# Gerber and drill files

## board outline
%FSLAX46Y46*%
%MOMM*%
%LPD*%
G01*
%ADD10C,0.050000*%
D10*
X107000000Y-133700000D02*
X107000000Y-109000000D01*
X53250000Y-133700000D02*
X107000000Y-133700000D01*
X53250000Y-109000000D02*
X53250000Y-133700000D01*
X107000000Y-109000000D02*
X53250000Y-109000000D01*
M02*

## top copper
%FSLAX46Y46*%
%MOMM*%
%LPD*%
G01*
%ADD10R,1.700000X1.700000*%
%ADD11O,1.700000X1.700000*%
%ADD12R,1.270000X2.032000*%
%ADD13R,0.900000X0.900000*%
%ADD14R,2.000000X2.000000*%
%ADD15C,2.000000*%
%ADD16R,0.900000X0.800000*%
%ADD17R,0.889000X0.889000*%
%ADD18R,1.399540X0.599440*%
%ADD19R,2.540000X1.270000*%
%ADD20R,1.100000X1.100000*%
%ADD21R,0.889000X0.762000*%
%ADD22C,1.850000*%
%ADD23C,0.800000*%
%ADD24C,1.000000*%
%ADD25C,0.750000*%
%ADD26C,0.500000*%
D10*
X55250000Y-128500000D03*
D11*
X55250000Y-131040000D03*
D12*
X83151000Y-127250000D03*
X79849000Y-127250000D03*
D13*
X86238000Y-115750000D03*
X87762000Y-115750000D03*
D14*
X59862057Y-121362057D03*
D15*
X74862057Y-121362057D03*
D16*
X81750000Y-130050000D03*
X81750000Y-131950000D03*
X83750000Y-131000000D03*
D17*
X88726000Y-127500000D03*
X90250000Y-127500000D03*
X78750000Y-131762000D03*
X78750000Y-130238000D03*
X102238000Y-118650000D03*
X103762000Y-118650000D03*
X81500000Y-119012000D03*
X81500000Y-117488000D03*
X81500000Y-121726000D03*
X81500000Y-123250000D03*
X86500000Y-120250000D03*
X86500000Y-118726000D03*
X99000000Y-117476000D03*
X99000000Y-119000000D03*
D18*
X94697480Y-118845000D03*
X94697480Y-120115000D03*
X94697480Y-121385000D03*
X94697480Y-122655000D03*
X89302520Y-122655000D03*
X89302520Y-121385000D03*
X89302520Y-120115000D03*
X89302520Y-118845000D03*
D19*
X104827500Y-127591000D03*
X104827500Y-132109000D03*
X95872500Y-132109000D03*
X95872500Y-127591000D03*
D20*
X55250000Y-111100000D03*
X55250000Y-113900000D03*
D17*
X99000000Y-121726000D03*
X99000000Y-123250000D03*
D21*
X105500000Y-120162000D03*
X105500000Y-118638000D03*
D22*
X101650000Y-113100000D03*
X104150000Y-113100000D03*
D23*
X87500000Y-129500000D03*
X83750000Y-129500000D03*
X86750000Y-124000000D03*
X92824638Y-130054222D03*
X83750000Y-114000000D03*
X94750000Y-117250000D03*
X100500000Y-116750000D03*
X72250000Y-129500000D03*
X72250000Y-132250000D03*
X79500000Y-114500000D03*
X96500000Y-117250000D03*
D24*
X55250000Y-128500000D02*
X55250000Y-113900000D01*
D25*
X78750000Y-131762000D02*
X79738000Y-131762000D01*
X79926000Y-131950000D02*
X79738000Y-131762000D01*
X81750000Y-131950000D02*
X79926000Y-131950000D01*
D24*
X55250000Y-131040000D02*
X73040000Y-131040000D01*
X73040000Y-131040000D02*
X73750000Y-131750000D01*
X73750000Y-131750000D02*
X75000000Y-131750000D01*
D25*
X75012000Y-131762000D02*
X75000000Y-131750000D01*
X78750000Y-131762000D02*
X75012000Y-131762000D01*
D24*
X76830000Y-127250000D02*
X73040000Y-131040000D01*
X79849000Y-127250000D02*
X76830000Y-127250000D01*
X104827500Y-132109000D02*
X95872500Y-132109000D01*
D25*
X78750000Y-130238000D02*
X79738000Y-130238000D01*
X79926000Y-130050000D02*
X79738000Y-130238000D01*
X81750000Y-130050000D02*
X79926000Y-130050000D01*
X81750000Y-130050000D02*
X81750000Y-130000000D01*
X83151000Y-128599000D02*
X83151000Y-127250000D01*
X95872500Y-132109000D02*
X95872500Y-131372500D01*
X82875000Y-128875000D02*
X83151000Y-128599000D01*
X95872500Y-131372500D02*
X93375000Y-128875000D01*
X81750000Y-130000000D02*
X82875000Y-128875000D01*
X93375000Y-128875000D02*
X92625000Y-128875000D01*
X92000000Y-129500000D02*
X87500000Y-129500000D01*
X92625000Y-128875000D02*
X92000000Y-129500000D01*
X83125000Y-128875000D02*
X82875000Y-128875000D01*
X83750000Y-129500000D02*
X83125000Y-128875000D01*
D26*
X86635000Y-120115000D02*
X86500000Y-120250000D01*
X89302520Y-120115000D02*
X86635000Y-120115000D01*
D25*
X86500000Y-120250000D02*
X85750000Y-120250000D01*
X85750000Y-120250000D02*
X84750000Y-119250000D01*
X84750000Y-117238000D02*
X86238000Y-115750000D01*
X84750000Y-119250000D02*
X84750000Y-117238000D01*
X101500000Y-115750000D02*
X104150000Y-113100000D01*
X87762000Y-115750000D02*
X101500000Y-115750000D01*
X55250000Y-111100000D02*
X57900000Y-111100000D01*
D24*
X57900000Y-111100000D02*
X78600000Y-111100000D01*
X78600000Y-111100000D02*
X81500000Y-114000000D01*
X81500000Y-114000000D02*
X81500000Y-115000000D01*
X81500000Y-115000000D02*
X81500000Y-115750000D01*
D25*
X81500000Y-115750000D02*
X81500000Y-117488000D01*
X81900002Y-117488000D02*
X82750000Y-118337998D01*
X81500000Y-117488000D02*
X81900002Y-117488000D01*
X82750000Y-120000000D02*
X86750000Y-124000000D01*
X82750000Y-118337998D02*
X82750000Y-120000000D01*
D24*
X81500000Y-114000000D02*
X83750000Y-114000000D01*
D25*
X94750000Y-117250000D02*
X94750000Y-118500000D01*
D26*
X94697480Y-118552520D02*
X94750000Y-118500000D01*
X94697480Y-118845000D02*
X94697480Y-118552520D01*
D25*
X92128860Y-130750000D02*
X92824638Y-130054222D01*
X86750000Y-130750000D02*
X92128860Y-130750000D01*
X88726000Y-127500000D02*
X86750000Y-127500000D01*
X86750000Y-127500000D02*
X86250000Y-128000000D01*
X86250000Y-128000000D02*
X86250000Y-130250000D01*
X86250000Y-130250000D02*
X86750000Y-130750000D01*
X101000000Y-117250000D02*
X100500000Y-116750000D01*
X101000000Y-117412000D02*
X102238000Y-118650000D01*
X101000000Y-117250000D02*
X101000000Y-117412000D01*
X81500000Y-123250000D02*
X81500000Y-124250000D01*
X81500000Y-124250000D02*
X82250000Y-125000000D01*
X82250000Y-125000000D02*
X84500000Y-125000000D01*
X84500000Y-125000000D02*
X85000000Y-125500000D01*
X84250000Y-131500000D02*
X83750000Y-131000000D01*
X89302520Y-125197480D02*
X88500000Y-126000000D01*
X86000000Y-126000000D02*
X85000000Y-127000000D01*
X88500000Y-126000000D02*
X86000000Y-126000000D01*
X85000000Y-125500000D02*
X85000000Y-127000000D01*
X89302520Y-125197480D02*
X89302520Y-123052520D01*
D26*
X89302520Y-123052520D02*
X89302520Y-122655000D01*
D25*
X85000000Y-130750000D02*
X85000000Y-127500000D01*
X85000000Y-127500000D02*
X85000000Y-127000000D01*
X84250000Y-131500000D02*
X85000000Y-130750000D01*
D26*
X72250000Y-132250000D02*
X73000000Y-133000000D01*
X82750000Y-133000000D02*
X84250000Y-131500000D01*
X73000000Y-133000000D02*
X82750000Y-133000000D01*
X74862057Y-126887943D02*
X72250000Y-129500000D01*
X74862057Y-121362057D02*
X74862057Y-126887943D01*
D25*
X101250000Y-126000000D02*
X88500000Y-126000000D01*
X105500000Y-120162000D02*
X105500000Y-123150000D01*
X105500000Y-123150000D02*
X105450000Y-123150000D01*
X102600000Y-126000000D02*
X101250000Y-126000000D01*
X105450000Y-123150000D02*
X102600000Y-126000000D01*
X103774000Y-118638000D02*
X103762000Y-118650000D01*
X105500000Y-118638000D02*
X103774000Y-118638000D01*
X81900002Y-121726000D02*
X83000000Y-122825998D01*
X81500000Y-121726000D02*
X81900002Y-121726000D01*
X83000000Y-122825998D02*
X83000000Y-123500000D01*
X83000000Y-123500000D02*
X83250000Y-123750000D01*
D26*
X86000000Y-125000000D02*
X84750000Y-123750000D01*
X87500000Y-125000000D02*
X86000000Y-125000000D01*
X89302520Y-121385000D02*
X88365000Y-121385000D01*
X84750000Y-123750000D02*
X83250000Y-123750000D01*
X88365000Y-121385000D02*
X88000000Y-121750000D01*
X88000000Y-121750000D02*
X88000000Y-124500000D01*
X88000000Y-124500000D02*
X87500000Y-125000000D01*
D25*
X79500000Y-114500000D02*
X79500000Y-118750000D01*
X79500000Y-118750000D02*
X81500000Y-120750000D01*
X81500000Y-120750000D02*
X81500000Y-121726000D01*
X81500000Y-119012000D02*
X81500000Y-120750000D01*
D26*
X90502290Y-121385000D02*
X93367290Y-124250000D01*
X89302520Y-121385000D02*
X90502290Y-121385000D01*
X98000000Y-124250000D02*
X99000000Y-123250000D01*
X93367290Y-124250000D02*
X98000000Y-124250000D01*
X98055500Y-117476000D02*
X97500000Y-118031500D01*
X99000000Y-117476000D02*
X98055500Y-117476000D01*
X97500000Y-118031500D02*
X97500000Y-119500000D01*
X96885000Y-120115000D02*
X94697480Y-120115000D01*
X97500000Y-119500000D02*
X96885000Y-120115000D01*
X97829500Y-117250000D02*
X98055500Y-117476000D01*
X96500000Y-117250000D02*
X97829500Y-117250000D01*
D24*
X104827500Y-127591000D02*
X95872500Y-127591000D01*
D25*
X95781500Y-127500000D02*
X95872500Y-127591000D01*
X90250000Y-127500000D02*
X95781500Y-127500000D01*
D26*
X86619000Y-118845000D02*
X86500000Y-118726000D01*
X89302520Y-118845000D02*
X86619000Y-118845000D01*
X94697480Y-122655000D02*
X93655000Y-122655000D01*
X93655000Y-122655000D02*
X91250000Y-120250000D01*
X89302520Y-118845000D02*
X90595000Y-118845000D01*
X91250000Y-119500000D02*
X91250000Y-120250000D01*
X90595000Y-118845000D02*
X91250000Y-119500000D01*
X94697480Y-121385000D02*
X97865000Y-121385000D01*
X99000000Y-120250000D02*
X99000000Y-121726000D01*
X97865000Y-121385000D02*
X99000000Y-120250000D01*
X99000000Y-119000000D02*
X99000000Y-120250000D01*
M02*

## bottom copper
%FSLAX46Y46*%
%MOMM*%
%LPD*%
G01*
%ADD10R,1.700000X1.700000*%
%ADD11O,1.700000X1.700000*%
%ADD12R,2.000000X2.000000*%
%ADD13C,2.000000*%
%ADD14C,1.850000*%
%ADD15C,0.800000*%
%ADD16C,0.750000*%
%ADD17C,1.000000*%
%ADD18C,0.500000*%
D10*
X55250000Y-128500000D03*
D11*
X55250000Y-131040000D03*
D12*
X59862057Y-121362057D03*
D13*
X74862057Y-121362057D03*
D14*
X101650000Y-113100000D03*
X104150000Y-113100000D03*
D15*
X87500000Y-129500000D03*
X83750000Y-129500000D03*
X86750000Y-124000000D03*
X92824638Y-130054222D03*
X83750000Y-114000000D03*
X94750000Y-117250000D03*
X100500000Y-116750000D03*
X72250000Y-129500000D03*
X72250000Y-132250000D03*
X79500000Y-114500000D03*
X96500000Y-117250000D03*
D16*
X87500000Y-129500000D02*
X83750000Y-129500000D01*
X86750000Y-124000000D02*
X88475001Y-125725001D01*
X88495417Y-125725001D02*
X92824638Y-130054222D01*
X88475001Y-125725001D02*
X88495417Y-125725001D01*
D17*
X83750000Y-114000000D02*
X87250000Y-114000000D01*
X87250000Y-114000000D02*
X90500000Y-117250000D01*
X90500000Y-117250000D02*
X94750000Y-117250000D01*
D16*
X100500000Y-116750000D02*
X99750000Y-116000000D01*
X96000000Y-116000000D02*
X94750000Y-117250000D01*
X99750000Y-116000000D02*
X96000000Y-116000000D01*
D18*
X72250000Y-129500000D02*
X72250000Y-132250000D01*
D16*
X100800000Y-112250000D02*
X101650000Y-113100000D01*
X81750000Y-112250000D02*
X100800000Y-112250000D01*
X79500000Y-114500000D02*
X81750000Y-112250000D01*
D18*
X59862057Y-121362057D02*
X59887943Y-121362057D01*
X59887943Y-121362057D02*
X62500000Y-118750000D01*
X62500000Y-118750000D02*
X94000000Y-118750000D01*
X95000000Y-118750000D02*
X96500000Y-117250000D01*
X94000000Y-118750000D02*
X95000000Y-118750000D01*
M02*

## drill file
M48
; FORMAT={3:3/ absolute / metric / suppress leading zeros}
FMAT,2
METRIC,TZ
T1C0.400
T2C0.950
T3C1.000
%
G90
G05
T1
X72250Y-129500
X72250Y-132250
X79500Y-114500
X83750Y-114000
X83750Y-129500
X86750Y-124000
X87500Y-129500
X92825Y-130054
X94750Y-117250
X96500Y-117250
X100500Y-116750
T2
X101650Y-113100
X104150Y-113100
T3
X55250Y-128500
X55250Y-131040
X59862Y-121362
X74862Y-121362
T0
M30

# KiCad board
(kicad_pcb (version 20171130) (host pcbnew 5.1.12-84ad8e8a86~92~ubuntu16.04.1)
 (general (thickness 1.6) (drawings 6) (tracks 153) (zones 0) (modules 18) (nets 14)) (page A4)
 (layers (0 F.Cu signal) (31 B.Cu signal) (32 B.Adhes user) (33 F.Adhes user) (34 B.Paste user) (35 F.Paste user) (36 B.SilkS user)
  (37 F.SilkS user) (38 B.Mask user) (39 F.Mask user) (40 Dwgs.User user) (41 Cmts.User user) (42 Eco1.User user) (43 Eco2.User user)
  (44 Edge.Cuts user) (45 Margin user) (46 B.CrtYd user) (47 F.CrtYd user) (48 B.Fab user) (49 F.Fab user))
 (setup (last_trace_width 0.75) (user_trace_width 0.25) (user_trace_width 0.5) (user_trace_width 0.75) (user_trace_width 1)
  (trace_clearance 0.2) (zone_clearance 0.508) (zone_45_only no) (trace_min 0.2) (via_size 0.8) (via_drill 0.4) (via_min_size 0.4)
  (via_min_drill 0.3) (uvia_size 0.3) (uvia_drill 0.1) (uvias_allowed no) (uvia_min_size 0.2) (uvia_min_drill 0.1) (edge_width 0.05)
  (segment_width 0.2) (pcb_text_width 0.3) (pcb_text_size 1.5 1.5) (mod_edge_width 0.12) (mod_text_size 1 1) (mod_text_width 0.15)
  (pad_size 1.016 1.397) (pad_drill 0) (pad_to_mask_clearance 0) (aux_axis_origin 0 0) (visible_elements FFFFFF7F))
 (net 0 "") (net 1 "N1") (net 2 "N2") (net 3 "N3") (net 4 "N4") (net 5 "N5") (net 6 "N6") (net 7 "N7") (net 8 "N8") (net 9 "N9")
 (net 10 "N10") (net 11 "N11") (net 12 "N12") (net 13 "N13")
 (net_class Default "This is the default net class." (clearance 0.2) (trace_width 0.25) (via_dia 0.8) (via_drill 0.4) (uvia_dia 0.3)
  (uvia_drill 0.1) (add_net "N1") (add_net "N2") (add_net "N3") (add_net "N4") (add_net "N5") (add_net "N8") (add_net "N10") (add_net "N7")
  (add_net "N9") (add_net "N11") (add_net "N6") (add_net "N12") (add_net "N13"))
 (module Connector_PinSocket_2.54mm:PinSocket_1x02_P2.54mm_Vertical (layer F.Cu) (at 55.25 128.5)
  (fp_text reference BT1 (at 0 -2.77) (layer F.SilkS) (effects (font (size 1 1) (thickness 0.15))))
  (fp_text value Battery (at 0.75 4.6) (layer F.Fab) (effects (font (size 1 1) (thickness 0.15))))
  (pad 1 thru_hole rect (at 0 0) (size 1.7 1.7) (drill 1) (layers *.Cu *.Mask) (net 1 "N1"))
  (pad 2 thru_hole oval (at 0 2.54) (size 1.7 1.7) (drill 1) (layers *.Cu *.Mask) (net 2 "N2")))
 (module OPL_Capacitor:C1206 (layer F.Cu) (at 81.5 127.25 180)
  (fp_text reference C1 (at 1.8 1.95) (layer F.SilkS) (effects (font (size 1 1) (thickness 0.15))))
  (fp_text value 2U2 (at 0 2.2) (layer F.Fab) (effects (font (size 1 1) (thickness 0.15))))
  (pad 1 smd rect (at -1.651 0 180) (size 1.27 2.032) (layers F.Cu F.Paste F.Mask) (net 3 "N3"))
  (pad 2 smd rect (at 1.651 0 180) (size 1.27 2.032) (layers F.Cu F.Paste F.Mask) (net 2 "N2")))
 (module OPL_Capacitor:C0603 (layer F.Cu) (at 87 115.75)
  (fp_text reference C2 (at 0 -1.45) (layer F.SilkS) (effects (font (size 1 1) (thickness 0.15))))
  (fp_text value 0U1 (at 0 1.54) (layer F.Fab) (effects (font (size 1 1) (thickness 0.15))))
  (pad 1 smd rect (at -0.762 0) (size 0.9 0.9) (layers F.Cu F.Paste F.Mask) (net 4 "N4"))
  (pad 2 smd rect (at 0.762 0) (size 0.9 0.9) (layers F.Cu F.Paste F.Mask) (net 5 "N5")))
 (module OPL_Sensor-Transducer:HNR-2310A (layer F.Cu) (at 59.862057 121.362057)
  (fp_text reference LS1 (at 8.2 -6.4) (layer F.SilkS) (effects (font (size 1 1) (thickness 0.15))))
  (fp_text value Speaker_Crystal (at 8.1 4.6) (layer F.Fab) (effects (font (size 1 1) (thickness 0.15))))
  (pad 1 thru_hole rect (at 0 0) (size 2 2) (drill 1) (layers *.Cu *.Mask) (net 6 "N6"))
  (pad 2 thru_hole circle (at 15 0) (size 2 2) (drill 1) (layers *.Cu *.Mask) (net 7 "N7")))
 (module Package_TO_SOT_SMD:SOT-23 (layer F.Cu) (at 82.75 131)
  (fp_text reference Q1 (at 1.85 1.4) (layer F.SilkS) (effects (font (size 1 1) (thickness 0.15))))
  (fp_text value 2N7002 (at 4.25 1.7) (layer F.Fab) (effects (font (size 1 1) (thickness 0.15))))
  (pad 1 smd rect (at -1 -0.95) (size 0.9 0.8) (layers F.Cu F.Paste F.Mask) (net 3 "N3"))
  (pad 2 smd rect (at -1 0.95) (size 0.9 0.8) (layers F.Cu F.Paste F.Mask) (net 2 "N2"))
  (pad 3 smd rect (at 1 0) (size 0.9 0.8) (layers F.Cu F.Paste F.Mask) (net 7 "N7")))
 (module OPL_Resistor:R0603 (layer F.Cu) (at 89.488 127.5)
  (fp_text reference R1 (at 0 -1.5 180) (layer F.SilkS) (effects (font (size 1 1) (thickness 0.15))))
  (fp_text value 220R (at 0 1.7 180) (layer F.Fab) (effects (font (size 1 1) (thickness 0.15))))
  (pad 1 smd rect (at -0.762 0) (size 0.889 0.889) (layers F.Cu F.Paste F.Mask) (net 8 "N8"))
  (pad 2 smd rect (at 0.762 0) (size 0.889 0.889) (layers F.Cu F.Paste F.Mask) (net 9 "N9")))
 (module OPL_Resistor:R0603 (layer F.Cu) (at 78.75 131 270)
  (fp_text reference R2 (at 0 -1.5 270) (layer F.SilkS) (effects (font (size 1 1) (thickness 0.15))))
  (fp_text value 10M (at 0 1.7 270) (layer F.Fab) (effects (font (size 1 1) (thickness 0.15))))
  (pad 2 smd rect (at 0.762 0 270) (size 0.889 0.889) (layers F.Cu F.Paste F.Mask) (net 2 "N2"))
  (pad 1 smd rect (at -0.762 0 270) (size 0.889 0.889) (layers F.Cu F.Paste F.Mask) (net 3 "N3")))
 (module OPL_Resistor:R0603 (layer F.Cu) (at 103 118.65)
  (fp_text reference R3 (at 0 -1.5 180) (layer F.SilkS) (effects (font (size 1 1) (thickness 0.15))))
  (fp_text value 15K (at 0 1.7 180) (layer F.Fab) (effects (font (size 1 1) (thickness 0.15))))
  (pad 1 smd rect (at -0.762 0) (size 0.889 0.889) (layers F.Cu F.Paste F.Mask) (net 8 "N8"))
  (pad 2 smd rect (at 0.762 0) (size 0.889 0.889) (layers F.Cu F.Paste F.Mask) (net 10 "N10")))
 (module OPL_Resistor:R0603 (layer F.Cu) (at 81.5 118.25 270)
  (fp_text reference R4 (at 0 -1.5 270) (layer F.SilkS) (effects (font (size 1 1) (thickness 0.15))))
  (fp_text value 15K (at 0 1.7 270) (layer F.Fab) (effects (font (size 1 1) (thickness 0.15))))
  (pad 2 smd rect (at 0.762 0 270) (size 0.889 0.889) (layers F.Cu F.Paste F.Mask) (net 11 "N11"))
  (pad 1 smd rect (at -0.762 0 270) (size 0.889 0.889) (layers F.Cu F.Paste F.Mask) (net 8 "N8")))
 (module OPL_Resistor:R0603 (layer F.Cu) (at 81.5 122.488 270)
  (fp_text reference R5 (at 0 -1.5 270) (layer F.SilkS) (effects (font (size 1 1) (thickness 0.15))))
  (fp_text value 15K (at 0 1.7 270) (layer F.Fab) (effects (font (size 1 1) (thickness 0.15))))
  (pad 1 smd rect (at -0.762 0 270) (size 0.889 0.889) (layers F.Cu F.Paste F.Mask) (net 11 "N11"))
  (pad 2 smd rect (at 0.762 0 270) (size 0.889 0.889) (layers F.Cu F.Paste F.Mask) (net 7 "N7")))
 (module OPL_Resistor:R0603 (layer F.Cu) (at 86.5 119.488 270)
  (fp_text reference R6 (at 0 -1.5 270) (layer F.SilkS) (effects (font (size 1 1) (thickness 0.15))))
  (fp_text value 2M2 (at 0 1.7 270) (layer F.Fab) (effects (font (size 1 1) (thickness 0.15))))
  (pad 2 smd rect (at 0.762 0 270) (size 0.889 0.889) (layers F.Cu F.Paste F.Mask) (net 4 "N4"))
  (pad 1 smd rect (at -0.762 0 270) (size 0.889 0.889) (layers F.Cu F.Paste F.Mask) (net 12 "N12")))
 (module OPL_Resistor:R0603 (layer F.Cu) (at 99 118.238 270)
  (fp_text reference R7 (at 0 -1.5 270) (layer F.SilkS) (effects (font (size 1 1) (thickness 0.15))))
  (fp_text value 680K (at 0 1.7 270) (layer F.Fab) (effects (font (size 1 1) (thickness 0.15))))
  (pad 1 smd rect (at -0.762 0 270) (size 0.889 0.889) (layers F.Cu F.Paste F.Mask) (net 6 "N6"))
  (pad 2 smd rect (at 0.762 0 270) (size 0.889 0.889) (layers F.Cu F.Paste F.Mask) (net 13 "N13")))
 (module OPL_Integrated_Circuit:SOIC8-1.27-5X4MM (layer F.Cu) (at 92 120.75)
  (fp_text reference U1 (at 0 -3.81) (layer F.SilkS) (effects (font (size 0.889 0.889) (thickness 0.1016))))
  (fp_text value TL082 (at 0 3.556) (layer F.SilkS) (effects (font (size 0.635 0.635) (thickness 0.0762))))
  (pad 8 smd rect (at 2.69748 -1.905) (size 1.39954 0.59944) (layers F.Cu F.Paste F.Mask) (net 8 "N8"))
  (pad 7 smd rect (at 2.69748 -0.635) (size 1.39954 0.59944) (layers F.Cu F.Paste F.Mask) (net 6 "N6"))
  (pad 6 smd rect (at 2.69748 0.635) (size 1.39954 0.59944) (layers F.Cu F.Paste F.Mask) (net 13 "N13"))
  (pad 5 smd rect (at 2.69748 1.905) (size 1.39954 0.59944) (layers F.Cu F.Paste F.Mask) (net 12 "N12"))
  (pad 4 smd rect (at -2.69748 1.905) (size 1.39954 0.59944) (layers F.Cu F.Paste F.Mask) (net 7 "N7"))
  (pad 3 smd rect (at -2.69748 0.635) (size 1.39954 0.59944) (layers F.Cu F.Paste F.Mask) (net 11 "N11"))
  (pad 2 smd rect (at -2.69748 -0.635) (size 1.39954 0.59944) (layers F.Cu F.Paste F.Mask) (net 4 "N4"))
  (pad 1 smd rect (at -2.69748 -1.905) (size 1.39954 0.59944) (layers F.Cu F.Paste F.Mask) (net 12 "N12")))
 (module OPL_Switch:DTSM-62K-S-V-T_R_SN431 (layer F.Cu) (at 100 129.75)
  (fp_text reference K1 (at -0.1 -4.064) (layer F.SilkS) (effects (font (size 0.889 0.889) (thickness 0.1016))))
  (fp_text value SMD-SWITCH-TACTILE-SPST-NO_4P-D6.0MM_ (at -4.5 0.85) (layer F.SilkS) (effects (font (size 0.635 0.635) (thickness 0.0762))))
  (pad 4 smd rect (at 4.8275 -2.159) (size 2.54 1.27) (layers F.Cu F.Paste F.Mask) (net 9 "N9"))
  (pad 3 smd rect (at 4.8275 2.359) (size 2.54 1.27) (layers F.Cu F.Paste F.Mask) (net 3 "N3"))
  (pad 2 smd rect (at -4.1275 2.359) (size 2.54 1.27) (layers F.Cu F.Paste F.Mask) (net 3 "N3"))
  (pad 1 smd rect (at -4.1275 -2.159) (size 2.54 1.27) (layers F.Cu F.Paste F.Mask) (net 9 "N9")))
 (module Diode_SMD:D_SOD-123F (layer F.Cu) (at 55.25 112.5 270)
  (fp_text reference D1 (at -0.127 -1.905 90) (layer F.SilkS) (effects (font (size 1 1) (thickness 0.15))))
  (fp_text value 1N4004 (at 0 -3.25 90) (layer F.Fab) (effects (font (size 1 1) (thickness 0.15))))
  (pad 1 smd rect (at -1.4 0 270) (size 1.1 1.1) (layers F.Cu F.Paste F.Mask) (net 8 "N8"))
  (pad 2 smd rect (at 1.4 0 270) (size 1.1 1.1) (layers F.Cu F.Paste F.Mask) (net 1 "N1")))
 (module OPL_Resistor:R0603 (layer F.Cu) (at 99 122.488 270)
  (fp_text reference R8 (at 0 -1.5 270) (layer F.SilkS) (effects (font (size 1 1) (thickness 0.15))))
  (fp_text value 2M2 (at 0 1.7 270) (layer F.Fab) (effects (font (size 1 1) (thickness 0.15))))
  (pad 1 smd rect (at -0.762 0 270) (size 0.889 0.889) (layers F.Cu F.Paste F.Mask) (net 13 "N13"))
  (pad 2 smd rect (at 0.762 0 270) (size 0.889 0.889) (layers F.Cu F.Paste F.Mask) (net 11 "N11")))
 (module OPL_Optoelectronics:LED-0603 (layer F.Cu) (at 105.5 119.4 270)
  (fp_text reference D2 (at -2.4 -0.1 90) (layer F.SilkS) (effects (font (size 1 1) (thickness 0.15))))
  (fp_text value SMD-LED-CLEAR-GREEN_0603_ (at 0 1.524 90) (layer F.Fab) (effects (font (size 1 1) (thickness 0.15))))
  (pad 2 smd rect (at 0.762 0 270) (size 0.762 0.889) (layers F.Cu F.Paste F.Mask) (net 7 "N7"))
  (pad 1 smd rect (at -0.762 0 270) (size 0.762 0.889) (layers F.Cu F.Paste F.Mask) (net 10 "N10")))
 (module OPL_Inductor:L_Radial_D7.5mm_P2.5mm (layer F.Cu) (at 100.9 113.1)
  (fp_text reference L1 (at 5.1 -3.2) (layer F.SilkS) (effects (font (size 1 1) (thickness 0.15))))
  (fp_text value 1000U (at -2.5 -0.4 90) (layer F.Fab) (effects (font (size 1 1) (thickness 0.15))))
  (pad 1 thru_hole circle (at 0.75 0) (size 1.85 1.85) (drill 0.95) (layers *.Cu *.Mask) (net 11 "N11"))
  (pad 2 thru_hole circle (at 3.25 0) (size 1.85 1.85) (drill 0.95) (layers *.Cu *.Mask) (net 5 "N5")))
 (gr_line (start 107 133.7) (end 107 109) (layer Edge.Cuts) (width 0.05))
 (gr_line (start 53.25 133.7) (end 107 133.7) (layer Edge.Cuts) (width 0.05))
 (gr_line (start 53.25 109) (end 53.25 133.7) (layer Edge.Cuts) (width 0.05))
 (gr_line (start 107 109) (end 53.25 109) (layer Edge.Cuts) (width 0.05))
 (segment (start 55.25 128.5) (end 55.25 113.9) (width 1) (layer F.Cu) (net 1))
 (segment (start 78.75 131.762) (end 79.738 131.762) (width 0.75) (layer F.Cu) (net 2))
 (segment (start 79.926 131.95) (end 79.738 131.762) (width 0.75) (layer F.Cu) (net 2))
 (segment (start 81.75 131.95) (end 79.926 131.95) (width 0.75) (layer F.Cu) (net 2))
 (segment (start 55.25 131.04) (end 73.04 131.04) (width 1) (layer F.Cu) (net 2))
 (segment (start 73.04 131.04) (end 73.75 131.75) (width 1) (layer F.Cu) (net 2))
 (segment (start 73.75 131.75) (end 75 131.75) (width 1) (layer F.Cu) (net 2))
 (segment (start 75.012 131.762) (end 75 131.75) (width 0.75) (layer F.Cu) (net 2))
 (segment (start 78.75 131.762) (end 75.012 131.762) (width 0.75) (layer F.Cu) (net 2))
 (segment (start 76.83 127.25) (end 73.04 131.04) (width 1) (layer F.Cu) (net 2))
 (segment (start 79.849 127.25) (end 76.83 127.25) (width 1) (layer F.Cu) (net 2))
 (segment (start 104.8275 132.109) (end 95.8725 132.109) (width 1) (layer F.Cu) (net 3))
 (segment (start 78.75 130.238) (end 79.738 130.238) (width 0.75) (layer F.Cu) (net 3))
 (segment (start 79.926 130.05) (end 79.738 130.238) (width 0.75) (layer F.Cu) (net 3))
 (segment (start 81.75 130.05) (end 79.926 130.05) (width 0.75) (layer F.Cu) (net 3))
 (segment (start 81.75 130.05) (end 81.75 130) (width 0.75) (layer F.Cu) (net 3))
 (segment (start 83.151 128.599) (end 83.151 127.25) (width 0.75) (layer F.Cu) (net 3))
 (segment (start 95.8725 132.109) (end 95.8725 131.3725) (width 0.75) (layer F.Cu) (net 3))
 (segment (start 82.875 128.875) (end 83.151 128.599) (width 0.75) (layer F.Cu) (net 3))
 (segment (start 95.8725 131.3725) (end 93.375 128.875) (width 0.75) (layer F.Cu) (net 3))
 (segment (start 81.75 130) (end 82.875 128.875) (width 0.75) (layer F.Cu) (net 3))
 (segment (start 93.375 128.875) (end 92.625 128.875) (width 0.75) (layer F.Cu) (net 3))
 (segment (start 92 129.5) (end 87.5 129.5) (width 0.75) (layer F.Cu) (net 3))
 (via (at 87.5 129.5) (size 0.8) (drill 0.4) (layers F.Cu B.Cu) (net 3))
 (segment (start 92.625 128.875) (end 92 129.5) (width 0.75) (layer F.Cu) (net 3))
 (via (at 83.75 129.5) (size 0.8) (drill 0.4) (layers F.Cu B.Cu) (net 3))
 (segment (start 87.5 129.5) (end 83.75 129.5) (width 0.75) (layer B.Cu) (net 3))
 (segment (start 83.125 128.875) (end 82.875 128.875) (width 0.75) (layer F.Cu) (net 3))
 (segment (start 83.75 129.5) (end 83.125 128.875) (width 0.75) (layer F.Cu) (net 3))
 (segment (start 86.635 120.115) (end 86.5 120.25) (width 0.5) (layer F.Cu) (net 4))
 (segment (start 89.30252 120.115) (end 86.635 120.115) (width 0.5) (layer F.Cu) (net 4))
 (segment (start 86.5 120.25) (end 85.75 120.25) (width 0.75) (layer F.Cu) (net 4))
 (segment (start 85.75 120.25) (end 84.75 119.25) (width 0.75) (layer F.Cu) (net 4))
 (segment (start 84.75 117.238) (end 86.238 115.75) (width 0.75) (layer F.Cu) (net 4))
 (segment (start 84.75 119.25) (end 84.75 117.238) (width 0.75) (layer F.Cu) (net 4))
 (segment (start 101.5 115.75) (end 104.15 113.1) (width 0.75) (layer F.Cu) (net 5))
 (segment (start 87.762 115.75) (end 101.5 115.75) (width 0.75) (layer F.Cu) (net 5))
 (segment (start 55.25 111.1) (end 57.9 111.1) (width 0.75) (layer F.Cu) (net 8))
 (segment (start 57.9 111.1) (end 78.6 111.1) (width 1) (layer F.Cu) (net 8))
 (segment (start 78.6 111.1) (end 81.5 114) (width 1) (layer F.Cu) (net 8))
 (segment (start 81.5 114) (end 81.5 115) (width 1) (layer F.Cu) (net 8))
 (segment (start 81.5 115) (end 81.5 115.75) (width 1) (layer F.Cu) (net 8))
 (segment (start 81.5 115.75) (end 81.5 117.488) (width 0.75) (layer F.Cu) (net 8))
 (segment (start 81.900002 117.488) (end 82.75 118.337998) (width 0.75) (layer F.Cu) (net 8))
 (segment (start 81.5 117.488) (end 81.900002 117.488) (width 0.75) (layer F.Cu) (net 8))
 (segment (start 82.75 120) (end 86.75 124) (width 0.75) (layer F.Cu) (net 8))
 (via (at 86.75 124) (size 0.8) (drill 0.4) (layers F.Cu B.Cu) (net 8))
 (segment (start 82.75 118.337998) (end 82.75 120) (width 0.75) (layer F.Cu) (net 8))
 (segment (start 86.75 124) (end 88.475001 125.725001) (width 0.75) (layer B.Cu) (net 8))
 (via (at 92.824638 130.054222) (size 0.8) (drill 0.4) (layers F.Cu B.Cu) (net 8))
 (segment (start 88.495417 125.725001) (end 92.824638 130.054222) (width 0.75) (layer B.Cu) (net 8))
 (segment (start 88.475001 125.725001) (end 88.495417 125.725001) (width 0.75) (layer B.Cu) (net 8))
 (via (at 83.75 114) (size 0.8) (drill 0.4) (layers F.Cu B.Cu) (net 8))
 (segment (start 81.5 114) (end 83.75 114) (width 1) (layer F.Cu) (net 8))
 (segment (start 83.75 114) (end 87.25 114) (width 1) (layer B.Cu) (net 8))
 (segment (start 87.25 114) (end 90.5 117.25) (width 1) (layer B.Cu) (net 8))
 (via (at 94.75 117.25) (size 0.8) (drill 0.4) (layers F.Cu B.Cu) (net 8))
 (segment (start 90.5 117.25) (end 94.75 117.25) (width 1) (layer B.Cu) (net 8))
 (segment (start 94.75 117.25) (end 94.75 118.5) (width 0.75) (layer F.Cu) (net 8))
 (segment (start 94.69748 118.55252) (end 94.75 118.5) (width 0.5) (layer F.Cu) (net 8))
 (segment (start 94.69748 118.845) (end 94.69748 118.55252) (width 0.5) (layer F.Cu) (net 8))
 (segment (start 92.12886 130.75) (end 92.824638 130.054222) (width 0.75) (layer F.Cu) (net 8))
 (segment (start 86.75 130.75) (end 92.12886 130.75) (width 0.75) (layer F.Cu) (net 8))
 (segment (start 88.726 127.5) (end 86.75 127.5) (width 0.75) (layer F.Cu) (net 8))
 (segment (start 86.75 127.5) (end 86.25 128) (width 0.75) (layer F.Cu) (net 8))
 (segment (start 86.25 128) (end 86.25 130.25) (width 0.75) (layer F.Cu) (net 8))
 (segment (start 86.25 130.25) (end 86.75 130.75) (width 0.75) (layer F.Cu) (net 8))
 (via (at 100.5 116.75) (size 0.8) (drill 0.4) (layers F.Cu B.Cu) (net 8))
 (segment (start 101 117.25) (end 100.5 116.75) (width 0.75) (layer F.Cu) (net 8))
 (segment (start 100.5 116.75) (end 99.75 116) (width 0.75) (layer B.Cu) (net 8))
 (segment (start 96 116) (end 94.75 117.25) (width 0.75) (layer B.Cu) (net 8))
 (segment (start 99.75 116) (end 96 116) (width 0.75) (layer B.Cu) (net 8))
 (segment (start 101 117.412) (end 102.238 118.65) (width 0.75) (layer F.Cu) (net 8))
 (segment (start 101 117.25) (end 101 117.412) (width 0.75) (layer F.Cu) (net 8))
 (segment (start 81.5 123.25) (end 81.5 124.25) (width 0.75) (layer F.Cu) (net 7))
 (segment (start 81.5 124.25) (end 82.25 125) (width 0.75) (layer F.Cu) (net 7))
 (segment (start 82.25 125) (end 84.5 125) (width 0.75) (layer F.Cu) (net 7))
 (segment (start 84.5 125) (end 85 125.5) (width 0.75) (layer F.Cu) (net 7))
 (segment (start 84.25 131.5) (end 83.75 131) (width 0.75) (layer F.Cu) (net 7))
 (segment (start 89.30252 125.19748) (end 88.5 126) (width 0.75) (layer F.Cu) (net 7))
 (segment (start 86 126) (end 85 127) (width 0.75) (layer F.Cu) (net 7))
 (segment (start 88.5 126) (end 86 126) (width 0.75) (layer F.Cu) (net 7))
 (segment (start 85 125.5) (end 85 127) (width 0.75) (layer F.Cu) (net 7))
 (segment (start 89.30252 125.19748) (end 89.30252 123.05252) (width 0.75) (layer F.Cu) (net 7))
 (segment (start 89.30252 123.05252) (end 89.30252 122.655) (width 0.5) (layer F.Cu) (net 7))
 (segment (start 85 130.75) (end 85 127.5) (width 0.75) (layer F.Cu) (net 7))
 (segment (start 85 127.5) (end 85 127) (width 0.75) (layer F.Cu) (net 7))
 (segment (start 84.25 131.5) (end 85 130.75) (width 0.75) (layer F.Cu) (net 7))
 (via (at 72.25 129.5) (size 0.8) (drill 0.4) (layers F.Cu B.Cu) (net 7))
 (via (at 72.25 132.25) (size 0.8) (drill 0.4) (layers F.Cu B.Cu) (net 7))
 (segment (start 72.25 132.25) (end 73 133) (width 0.5) (layer F.Cu) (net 7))
 (segment (start 82.75 133) (end 84.25 131.5) (width 0.5) (layer F.Cu) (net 7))
 (segment (start 73 133) (end 82.75 133) (width 0.5) (layer F.Cu) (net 7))
 (segment (start 74.862057 126.887943) (end 72.25 129.5) (width 0.5) (layer F.Cu) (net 7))
 (segment (start 74.862057 121.362057) (end 74.862057 126.887943) (width 0.5) (layer F.Cu) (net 7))
 (segment (start 72.25 129.5) (end 72.25 132.25) (width 0.5) (layer B.Cu) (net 7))
 (segment (start 101.25 126) (end 88.5 126) (width 0.75) (layer F.Cu) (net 7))
 (segment (start 105.5 120.162) (end 105.5 123.15) (width 0.75) (layer F.Cu) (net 7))
 (segment (start 105.5 123.15) (end 105.45 123.15) (width 0.75) (layer F.Cu) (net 7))
 (segment (start 102.6 126) (end 101.25 126) (width 0.75) (layer F.Cu) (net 7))
 (segment (start 105.45 123.15) (end 102.6 126) (width 0.75) (layer F.Cu) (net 7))
 (segment (start 103.774 118.638) (end 103.762 118.65) (width 0.75) (layer F.Cu) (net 10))
 (segment (start 105.5 118.638) (end 103.774 118.638) (width 0.75) (layer F.Cu) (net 10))
 (segment (start 81.900002 121.726) (end 83 122.825998) (width 0.75) (layer F.Cu) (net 11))
 (segment (start 81.5 121.726) (end 81.900002 121.726) (width 0.75) (layer F.Cu) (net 11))
 (segment (start 83 122.825998) (end 83 123.5) (width 0.75) (layer F.Cu) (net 11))
 (segment (start 83 123.5) (end 83.25 123.75) (width 0.75) (layer F.Cu) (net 11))
 (segment (start 86 125) (end 84.75 123.75) (width 0.5) (layer F.Cu) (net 11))
 (segment (start 87.5 125) (end 86 125) (width 0.5) (layer F.Cu) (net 11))
 (segment (start 89.30252 121.385) (end 88.365 121.385) (width 0.5) (layer F.Cu) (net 11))
 (segment (start 84.75 123.75) (end 83.25 123.75) (width 0.5) (layer F.Cu) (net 11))
 (segment (start 88.365 121.385) (end 88 121.75) (width 0.5) (layer F.Cu) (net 11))
 (segment (start 88 121.75) (end 88 124.5) (width 0.5) (layer F.Cu) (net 11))
 (segment (start 88 124.5) (end 87.5 125) (width 0.5) (layer F.Cu) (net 11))
 (via (at 79.5 114.5) (size 0.8) (drill 0.4) (layers F.Cu B.Cu) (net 11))
 (segment (start 79.5 114.5) (end 79.5 118.75) (width 0.75) (layer F.Cu) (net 11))
 (segment (start 79.5 118.75) (end 81.5 120.75) (width 0.75) (layer F.Cu) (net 11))
 (segment (start 81.5 120.75) (end 81.5 121.726) (width 0.75) (layer F.Cu) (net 11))
 (segment (start 81.5 119.012) (end 81.5 120.75) (width 0.75) (layer F.Cu) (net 11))
 (segment (start 90.50229 121.385) (end 93.36729 124.25) (width 0.5) (layer F.Cu) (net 11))
 (segment (start 89.30252 121.385) (end 90.50229 121.385) (width 0.5) (layer F.Cu) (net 11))
 (segment (start 98 124.25) (end 99 123.25) (width 0.5) (layer F.Cu) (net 11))
 (segment (start 93.36729 124.25) (end 98 124.25) (width 0.5) (layer F.Cu) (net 11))
 (segment (start 100.8 112.25) (end 101.65 113.1) (width 0.75) (layer B.Cu) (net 11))
 (segment (start 81.75 112.25) (end 100.8 112.25) (width 0.75) (layer B.Cu) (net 11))
 (segment (start 79.5 114.5) (end 81.75 112.25) (width 0.75) (layer B.Cu) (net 11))
 (segment (start 98.0555 117.476) (end 97.5 118.0315) (width 0.5) (layer F.Cu) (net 6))
 (segment (start 99 117.476) (end 98.0555 117.476) (width 0.5) (layer F.Cu) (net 6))
 (segment (start 97.5 118.0315) (end 97.5 119.5) (width 0.5) (layer F.Cu) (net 6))
 (segment (start 96.885 120.115) (end 94.69748 120.115) (width 0.5) (layer F.Cu) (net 6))
 (segment (start 97.5 119.5) (end 96.885 120.115) (width 0.5) (layer F.Cu) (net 6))
 (segment (start 59.862057 121.362057) (end 59.887943 121.362057) (width 0.5) (layer B.Cu) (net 6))
 (segment (start 59.887943 121.362057) (end 62.5 118.75) (width 0.5) (layer B.Cu) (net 6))
 (segment (start 62.5 118.75) (end 94 118.75) (width 0.5) (layer B.Cu) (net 6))
 (via (at 96.5 117.25) (size 0.8) (drill 0.4) (layers F.Cu B.Cu) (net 6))
 (segment (start 95 118.75) (end 96.5 117.25) (width 0.5) (layer B.Cu) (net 6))
 (segment (start 94 118.75) (end 95 118.75) (width 0.5) (layer B.Cu) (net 6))
 (segment (start 97.8295 117.25) (end 98.0555 117.476) (width 0.5) (layer F.Cu) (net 6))
 (segment (start 96.5 117.25) (end 97.8295 117.25) (width 0.5) (layer F.Cu) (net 6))
 (segment (start 104.8275 127.591) (end 95.8725 127.591) (width 1) (layer F.Cu) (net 9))
 (segment (start 95.7815 127.5) (end 95.8725 127.591) (width 0.75) (layer F.Cu) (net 9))
 (segment (start 90.25 127.5) (end 95.7815 127.5) (width 0.75) (layer F.Cu) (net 9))
 (segment (start 86.619 118.845) (end 86.5 118.726) (width 0.5) (layer F.Cu) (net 12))
 (segment (start 89.30252 118.845) (end 86.619 118.845) (width 0.5) (layer F.Cu) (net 12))
 (segment (start 94.69748 122.655) (end 93.655 122.655) (width 0.5) (layer F.Cu) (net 12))
 (segment (start 93.655 122.655) (end 91.25 120.25) (width 0.5) (layer F.Cu) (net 12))
 (segment (start 89.30252 118.845) (end 90.595 118.845) (width 0.5) (layer F.Cu) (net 12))
 (segment (start 91.25 119.5) (end 91.25 120.25) (width 0.5) (layer F.Cu) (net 12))
 (segment (start 90.595 118.845) (end 91.25 119.5) (width 0.5) (layer F.Cu) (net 12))
 (segment (start 94.69748 121.385) (end 97.865 121.385) (width 0.5) (layer F.Cu) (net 13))
 (segment (start 99 120.25) (end 99 121.726) (width 0.5) (layer F.Cu) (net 13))
 (segment (start 97.865 121.385) (end 99 120.25) (width 0.5) (layer F.Cu) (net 13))
 (segment (start 99 119) (end 99 120.25) (width 0.5) (layer F.Cu) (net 13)))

